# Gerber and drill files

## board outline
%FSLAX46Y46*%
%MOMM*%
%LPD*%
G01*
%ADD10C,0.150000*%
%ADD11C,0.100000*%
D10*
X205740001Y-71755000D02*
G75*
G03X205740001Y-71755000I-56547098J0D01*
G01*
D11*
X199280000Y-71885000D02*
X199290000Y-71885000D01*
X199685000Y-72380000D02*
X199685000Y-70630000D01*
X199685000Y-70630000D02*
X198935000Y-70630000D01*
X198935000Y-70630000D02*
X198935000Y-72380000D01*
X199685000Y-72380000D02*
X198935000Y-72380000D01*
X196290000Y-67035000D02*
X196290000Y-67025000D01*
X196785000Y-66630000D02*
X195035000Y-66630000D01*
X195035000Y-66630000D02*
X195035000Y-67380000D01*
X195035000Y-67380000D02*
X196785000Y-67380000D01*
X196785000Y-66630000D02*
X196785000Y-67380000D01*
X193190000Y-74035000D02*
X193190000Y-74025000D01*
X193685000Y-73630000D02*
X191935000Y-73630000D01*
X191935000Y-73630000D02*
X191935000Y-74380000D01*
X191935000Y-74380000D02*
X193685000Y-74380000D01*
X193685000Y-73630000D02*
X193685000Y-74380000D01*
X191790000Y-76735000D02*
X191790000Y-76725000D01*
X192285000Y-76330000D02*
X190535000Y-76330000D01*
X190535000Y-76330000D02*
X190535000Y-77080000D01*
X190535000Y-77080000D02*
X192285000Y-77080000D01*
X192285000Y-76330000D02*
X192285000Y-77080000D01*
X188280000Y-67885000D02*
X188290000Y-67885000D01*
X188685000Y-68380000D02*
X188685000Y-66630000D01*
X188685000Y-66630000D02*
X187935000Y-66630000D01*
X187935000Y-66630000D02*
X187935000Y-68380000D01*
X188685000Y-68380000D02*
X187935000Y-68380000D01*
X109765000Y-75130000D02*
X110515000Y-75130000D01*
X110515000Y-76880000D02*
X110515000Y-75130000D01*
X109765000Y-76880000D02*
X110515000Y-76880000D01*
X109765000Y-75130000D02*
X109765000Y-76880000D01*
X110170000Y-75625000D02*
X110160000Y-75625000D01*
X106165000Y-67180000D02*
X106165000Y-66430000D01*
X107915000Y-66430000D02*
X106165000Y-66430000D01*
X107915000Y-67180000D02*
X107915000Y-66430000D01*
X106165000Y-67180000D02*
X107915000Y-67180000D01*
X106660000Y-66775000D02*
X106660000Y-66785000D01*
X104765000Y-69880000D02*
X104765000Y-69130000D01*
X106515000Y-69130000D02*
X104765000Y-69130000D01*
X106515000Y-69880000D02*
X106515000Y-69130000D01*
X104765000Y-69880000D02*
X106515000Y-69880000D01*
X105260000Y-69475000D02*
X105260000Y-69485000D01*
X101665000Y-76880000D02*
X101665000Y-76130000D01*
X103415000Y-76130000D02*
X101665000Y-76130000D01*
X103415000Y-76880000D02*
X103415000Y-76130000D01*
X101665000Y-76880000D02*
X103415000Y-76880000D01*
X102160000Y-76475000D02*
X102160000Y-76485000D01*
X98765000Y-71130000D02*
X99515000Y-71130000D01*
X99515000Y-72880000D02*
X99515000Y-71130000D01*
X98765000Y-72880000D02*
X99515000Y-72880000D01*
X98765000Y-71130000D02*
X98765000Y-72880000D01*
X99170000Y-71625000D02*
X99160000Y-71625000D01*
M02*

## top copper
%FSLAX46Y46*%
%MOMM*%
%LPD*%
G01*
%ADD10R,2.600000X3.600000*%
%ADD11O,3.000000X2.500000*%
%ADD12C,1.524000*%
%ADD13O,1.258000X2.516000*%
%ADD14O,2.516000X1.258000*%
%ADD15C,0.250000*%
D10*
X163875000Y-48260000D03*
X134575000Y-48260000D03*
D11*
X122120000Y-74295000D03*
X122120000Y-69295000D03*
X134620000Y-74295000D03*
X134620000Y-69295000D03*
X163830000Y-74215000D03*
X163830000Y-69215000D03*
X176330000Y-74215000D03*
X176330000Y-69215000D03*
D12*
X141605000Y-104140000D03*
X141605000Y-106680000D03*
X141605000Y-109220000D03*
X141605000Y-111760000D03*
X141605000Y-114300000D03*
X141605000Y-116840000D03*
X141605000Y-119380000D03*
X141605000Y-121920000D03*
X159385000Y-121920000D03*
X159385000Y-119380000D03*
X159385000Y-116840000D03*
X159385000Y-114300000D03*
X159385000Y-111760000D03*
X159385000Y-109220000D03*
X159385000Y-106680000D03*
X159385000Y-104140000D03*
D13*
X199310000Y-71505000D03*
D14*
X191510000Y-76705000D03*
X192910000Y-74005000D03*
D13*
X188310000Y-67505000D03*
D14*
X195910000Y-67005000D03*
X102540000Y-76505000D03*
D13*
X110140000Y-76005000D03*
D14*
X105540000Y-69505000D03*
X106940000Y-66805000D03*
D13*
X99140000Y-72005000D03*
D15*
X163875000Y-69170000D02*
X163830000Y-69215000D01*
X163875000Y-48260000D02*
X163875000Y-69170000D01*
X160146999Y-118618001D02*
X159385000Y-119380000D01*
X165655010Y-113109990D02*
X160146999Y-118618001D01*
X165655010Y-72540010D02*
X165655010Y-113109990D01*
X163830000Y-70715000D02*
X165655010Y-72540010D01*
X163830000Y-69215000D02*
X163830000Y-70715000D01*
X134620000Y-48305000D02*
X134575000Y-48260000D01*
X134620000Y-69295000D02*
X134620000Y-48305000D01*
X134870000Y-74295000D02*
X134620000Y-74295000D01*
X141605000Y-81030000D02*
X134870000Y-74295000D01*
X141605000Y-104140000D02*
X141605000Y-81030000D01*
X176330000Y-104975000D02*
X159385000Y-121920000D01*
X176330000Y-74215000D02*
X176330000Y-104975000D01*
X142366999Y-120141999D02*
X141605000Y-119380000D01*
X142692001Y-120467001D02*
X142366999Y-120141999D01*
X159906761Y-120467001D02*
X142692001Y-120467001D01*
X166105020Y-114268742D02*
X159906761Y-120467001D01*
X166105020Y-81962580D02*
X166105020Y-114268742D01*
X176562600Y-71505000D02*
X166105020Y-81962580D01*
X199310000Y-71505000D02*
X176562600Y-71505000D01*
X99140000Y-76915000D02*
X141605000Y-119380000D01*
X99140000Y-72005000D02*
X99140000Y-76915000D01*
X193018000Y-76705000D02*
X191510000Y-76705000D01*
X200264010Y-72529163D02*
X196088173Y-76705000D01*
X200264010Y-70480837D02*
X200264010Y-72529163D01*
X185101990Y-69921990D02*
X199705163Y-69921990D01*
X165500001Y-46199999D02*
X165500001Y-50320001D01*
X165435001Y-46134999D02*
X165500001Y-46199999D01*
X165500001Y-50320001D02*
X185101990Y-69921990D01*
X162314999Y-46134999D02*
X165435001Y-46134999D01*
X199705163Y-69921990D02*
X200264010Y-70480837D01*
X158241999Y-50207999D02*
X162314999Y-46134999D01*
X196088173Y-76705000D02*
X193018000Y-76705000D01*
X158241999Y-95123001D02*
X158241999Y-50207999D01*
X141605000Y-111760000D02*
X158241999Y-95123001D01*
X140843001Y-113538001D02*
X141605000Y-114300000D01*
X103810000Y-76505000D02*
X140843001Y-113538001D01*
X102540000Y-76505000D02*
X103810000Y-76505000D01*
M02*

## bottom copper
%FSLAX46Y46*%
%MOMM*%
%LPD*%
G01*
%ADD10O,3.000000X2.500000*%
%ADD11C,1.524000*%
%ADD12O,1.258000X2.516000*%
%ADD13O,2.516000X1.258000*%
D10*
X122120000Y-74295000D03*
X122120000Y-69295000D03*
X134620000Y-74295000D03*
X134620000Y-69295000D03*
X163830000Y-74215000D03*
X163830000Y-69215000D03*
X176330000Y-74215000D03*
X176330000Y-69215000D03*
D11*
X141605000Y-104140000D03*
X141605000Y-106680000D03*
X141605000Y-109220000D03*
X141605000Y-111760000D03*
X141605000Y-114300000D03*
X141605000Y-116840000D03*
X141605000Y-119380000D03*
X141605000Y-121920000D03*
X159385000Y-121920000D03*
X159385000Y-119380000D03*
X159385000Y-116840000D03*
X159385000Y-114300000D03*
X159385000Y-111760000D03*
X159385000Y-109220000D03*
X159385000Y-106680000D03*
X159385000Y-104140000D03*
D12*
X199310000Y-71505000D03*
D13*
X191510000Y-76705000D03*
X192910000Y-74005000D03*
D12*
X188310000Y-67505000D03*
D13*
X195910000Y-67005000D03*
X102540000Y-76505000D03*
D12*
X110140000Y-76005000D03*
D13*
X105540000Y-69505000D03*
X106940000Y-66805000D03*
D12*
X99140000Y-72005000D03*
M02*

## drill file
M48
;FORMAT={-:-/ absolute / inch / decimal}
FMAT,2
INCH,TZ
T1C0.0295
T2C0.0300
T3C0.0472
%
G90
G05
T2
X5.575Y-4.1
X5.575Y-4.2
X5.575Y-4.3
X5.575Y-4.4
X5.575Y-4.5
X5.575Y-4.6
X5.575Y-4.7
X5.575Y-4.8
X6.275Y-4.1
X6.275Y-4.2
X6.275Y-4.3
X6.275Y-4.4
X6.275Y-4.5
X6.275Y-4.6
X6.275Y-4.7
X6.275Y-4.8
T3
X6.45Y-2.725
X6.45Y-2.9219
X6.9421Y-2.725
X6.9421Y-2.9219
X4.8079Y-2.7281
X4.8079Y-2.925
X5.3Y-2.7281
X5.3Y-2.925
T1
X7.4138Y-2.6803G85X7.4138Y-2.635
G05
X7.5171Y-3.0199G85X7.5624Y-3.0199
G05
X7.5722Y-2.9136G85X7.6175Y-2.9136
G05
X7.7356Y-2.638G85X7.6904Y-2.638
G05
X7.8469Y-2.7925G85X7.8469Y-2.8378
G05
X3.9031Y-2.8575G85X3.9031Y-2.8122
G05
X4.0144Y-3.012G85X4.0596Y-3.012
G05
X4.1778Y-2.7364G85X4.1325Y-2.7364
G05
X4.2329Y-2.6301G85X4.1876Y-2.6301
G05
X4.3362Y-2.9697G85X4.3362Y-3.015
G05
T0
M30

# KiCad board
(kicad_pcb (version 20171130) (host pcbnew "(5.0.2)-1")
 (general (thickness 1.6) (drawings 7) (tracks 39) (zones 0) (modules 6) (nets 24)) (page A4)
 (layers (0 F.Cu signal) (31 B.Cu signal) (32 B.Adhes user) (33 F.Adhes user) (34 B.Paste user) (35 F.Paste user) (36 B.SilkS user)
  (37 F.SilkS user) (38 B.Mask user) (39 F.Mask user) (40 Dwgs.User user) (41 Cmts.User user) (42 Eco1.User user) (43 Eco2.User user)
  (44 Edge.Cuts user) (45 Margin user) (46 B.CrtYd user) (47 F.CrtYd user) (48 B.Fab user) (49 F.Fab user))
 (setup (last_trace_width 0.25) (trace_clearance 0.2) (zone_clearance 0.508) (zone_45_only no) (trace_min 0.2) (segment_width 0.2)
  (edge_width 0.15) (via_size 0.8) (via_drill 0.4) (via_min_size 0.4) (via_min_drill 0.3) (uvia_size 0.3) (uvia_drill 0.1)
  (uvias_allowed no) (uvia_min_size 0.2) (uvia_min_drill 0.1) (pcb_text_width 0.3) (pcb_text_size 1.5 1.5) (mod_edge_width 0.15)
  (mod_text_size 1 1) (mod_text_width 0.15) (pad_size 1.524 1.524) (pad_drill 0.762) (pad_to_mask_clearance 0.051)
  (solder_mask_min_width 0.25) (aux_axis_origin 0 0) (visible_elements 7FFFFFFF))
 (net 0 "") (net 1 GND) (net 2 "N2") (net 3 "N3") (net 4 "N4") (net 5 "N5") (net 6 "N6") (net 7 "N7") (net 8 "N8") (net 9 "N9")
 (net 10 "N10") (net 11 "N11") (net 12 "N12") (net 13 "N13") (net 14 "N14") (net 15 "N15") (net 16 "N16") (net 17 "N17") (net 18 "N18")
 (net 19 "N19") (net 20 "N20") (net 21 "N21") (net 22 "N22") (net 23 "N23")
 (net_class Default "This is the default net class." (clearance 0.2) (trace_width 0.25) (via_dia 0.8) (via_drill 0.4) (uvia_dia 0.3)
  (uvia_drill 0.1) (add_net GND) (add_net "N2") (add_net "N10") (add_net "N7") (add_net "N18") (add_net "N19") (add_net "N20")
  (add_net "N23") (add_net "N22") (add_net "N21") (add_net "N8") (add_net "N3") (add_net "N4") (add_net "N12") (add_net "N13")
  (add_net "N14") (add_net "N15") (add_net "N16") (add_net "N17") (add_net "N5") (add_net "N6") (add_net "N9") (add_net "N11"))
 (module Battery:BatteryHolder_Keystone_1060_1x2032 (layer F.Cu) (at 149.225 48.26)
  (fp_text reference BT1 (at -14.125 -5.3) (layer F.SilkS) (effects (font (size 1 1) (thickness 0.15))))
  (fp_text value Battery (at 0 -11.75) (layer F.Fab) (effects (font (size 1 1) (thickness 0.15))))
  (pad 2 smd rect (at 14.65 0 180) (size 2.6 3.6) (layers F.Cu F.Paste F.Mask) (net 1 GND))
  (pad 1 smd rect (at -14.65 0 180) (size 2.6 3.6) (layers F.Cu F.Paste F.Mask) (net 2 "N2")))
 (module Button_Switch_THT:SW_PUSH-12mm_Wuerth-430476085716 (layer F.Cu) (at 134.62 74.295 180)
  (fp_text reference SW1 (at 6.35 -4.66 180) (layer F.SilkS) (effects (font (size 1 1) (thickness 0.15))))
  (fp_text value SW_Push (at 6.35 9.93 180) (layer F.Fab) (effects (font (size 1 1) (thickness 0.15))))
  (pad 1 thru_hole oval (at 12.5 0 180) (size 3 2.5) (drill 1.2) (layers *.Cu *.Mask) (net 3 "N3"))
  (pad 2 thru_hole oval (at 12.5 5 180) (size 3 2.5) (drill 1.2) (layers *.Cu *.Mask) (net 2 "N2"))
  (pad 1 thru_hole oval (at 0 0 180) (size 3 2.5) (drill 1.2) (layers *.Cu *.Mask) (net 3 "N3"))
  (pad 2 thru_hole oval (at 0 5 180) (size 3 2.5) (drill 1.2) (layers *.Cu *.Mask) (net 2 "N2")))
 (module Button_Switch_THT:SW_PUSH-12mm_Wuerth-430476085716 (layer F.Cu) (at 163.83 69.215)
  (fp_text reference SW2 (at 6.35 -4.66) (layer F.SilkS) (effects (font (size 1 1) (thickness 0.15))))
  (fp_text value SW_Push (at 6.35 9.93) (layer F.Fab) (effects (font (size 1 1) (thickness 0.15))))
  (pad 2 thru_hole oval (at 0 5) (size 3 2.5) (drill 1.2) (layers *.Cu *.Mask) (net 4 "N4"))
  (pad 1 thru_hole oval (at 0 0) (size 3 2.5) (drill 1.2) (layers *.Cu *.Mask) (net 1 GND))
  (pad 2 thru_hole oval (at 12.5 5) (size 3 2.5) (drill 1.2) (layers *.Cu *.Mask) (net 4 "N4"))
  (pad 1 thru_hole oval (at 12.5 0) (size 3 2.5) (drill 1.2) (layers *.Cu *.Mask) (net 1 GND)))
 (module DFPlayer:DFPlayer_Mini (layer F.Cu) (at 150.495 101.6)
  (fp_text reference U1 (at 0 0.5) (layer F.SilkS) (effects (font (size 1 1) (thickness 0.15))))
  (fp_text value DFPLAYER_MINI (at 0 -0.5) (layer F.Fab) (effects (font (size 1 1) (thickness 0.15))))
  (pad 1 thru_hole circle (at -8.89 2.54) (size 1.524 1.524) (drill 0.762) (layers *.Cu *.Mask) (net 3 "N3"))
  (pad 2 thru_hole circle (at -8.89 5.08) (size 1.524 1.524) (drill 0.762) (layers *.Cu *.Mask) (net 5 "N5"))
  (pad 3 thru_hole circle (at -8.89 7.62) (size 1.524 1.524) (drill 0.762) (layers *.Cu *.Mask) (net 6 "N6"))
  (pad 4 thru_hole circle (at -8.89 10.16) (size 1.524 1.524) (drill 0.762) (layers *.Cu *.Mask) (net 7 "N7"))
  (pad 5 thru_hole circle (at -8.89 12.7) (size 1.524 1.524) (drill 0.762) (layers *.Cu *.Mask) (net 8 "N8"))
  (pad 6 thru_hole circle (at -8.89 15.24) (size 1.524 1.524) (drill 0.762) (layers *.Cu *.Mask) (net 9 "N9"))
  (pad 7 thru_hole circle (at -8.89 17.78) (size 1.524 1.524) (drill 0.762) (layers *.Cu *.Mask) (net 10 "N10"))
  (pad 8 thru_hole circle (at -8.89 20.32) (size 1.524 1.524) (drill 0.762) (layers *.Cu *.Mask) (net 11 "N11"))
  (pad 9 thru_hole circle (at 8.89 20.32) (size 1.524 1.524) (drill 0.762) (layers *.Cu *.Mask) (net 4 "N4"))
  (pad 10 thru_hole circle (at 8.89 17.78) (size 1.524 1.524) (drill 0.762) (layers *.Cu *.Mask) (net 1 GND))
  (pad 11 thru_hole circle (at 8.89 15.24) (size 1.524 1.524) (drill 0.762) (layers *.Cu *.Mask) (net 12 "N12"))
  (pad 12 thru_hole circle (at 8.89 12.7) (size 1.524 1.524) (drill 0.762) (layers *.Cu *.Mask) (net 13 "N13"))
  (pad 13 thru_hole circle (at 8.89 10.16) (size 1.524 1.524) (drill 0.762) (layers *.Cu *.Mask) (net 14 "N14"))
  (pad 14 thru_hole circle (at 8.89 7.62) (size 1.524 1.524) (drill 0.762) (layers *.Cu *.Mask) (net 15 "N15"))
  (pad 15 thru_hole circle (at 8.89 5.08) (size 1.524 1.524) (drill 0.762) (layers *.Cu *.Mask) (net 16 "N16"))
  (pad 16 thru_hole circle (at 8.89 2.54) (size 1.524 1.524) (drill 0.762) (layers *.Cu *.Mask) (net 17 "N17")))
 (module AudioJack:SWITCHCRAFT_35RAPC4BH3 (layer F.Cu) (at 194.31 71.755 180)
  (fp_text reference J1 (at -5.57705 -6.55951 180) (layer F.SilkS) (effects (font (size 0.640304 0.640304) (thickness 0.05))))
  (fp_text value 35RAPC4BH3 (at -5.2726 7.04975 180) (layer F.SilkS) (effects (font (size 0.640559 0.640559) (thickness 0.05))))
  (fp_line (start -4.97 -0.13) (end -4.98 -0.13) (layer Edge.Cuts) (width 0.1))
  (fp_line (start -5.375 -0.625) (end -5.375 1.125) (layer Edge.Cuts) (width 0.1))
  (fp_line (start -5.375 1.125) (end -4.625 1.125) (layer Edge.Cuts) (width 0.1))
  (fp_line (start -4.625 1.125) (end -4.625 -0.625) (layer Edge.Cuts) (width 0.1))
  (fp_line (start -5.375 -0.625) (end -4.625 -0.625) (layer Edge.Cuts) (width 0.1))
  (fp_line (start -1.98 4.72) (end -1.98 4.73) (layer Edge.Cuts) (width 0.1))
  (fp_line (start -2.475 5.125) (end -0.725 5.125) (layer Edge.Cuts) (width 0.1))
  (fp_line (start -0.725 5.125) (end -0.725 4.375) (layer Edge.Cuts) (width 0.1))
  (fp_line (start -0.725 4.375) (end -2.475 4.375) (layer Edge.Cuts) (width 0.1))
  (fp_line (start -2.475 5.125) (end -2.475 4.375) (layer Edge.Cuts) (width 0.1))
  (fp_line (start 1.12 -2.28) (end 1.12 -2.27) (layer Edge.Cuts) (width 0.1))
  (fp_line (start 0.625 -1.875) (end 2.375 -1.875) (layer Edge.Cuts) (width 0.1))
  (fp_line (start 2.375 -1.875) (end 2.375 -2.625) (layer Edge.Cuts) (width 0.1))
  (fp_line (start 2.375 -2.625) (end 0.625 -2.625) (layer Edge.Cuts) (width 0.1))
  (fp_line (start 0.625 -1.875) (end 0.625 -2.625) (layer Edge.Cuts) (width 0.1))
  (fp_line (start 2.52 -4.98) (end 2.52 -4.97) (layer Edge.Cuts) (width 0.1))
  (fp_line (start 2.025 -4.575) (end 3.775 -4.575) (layer Edge.Cuts) (width 0.1))
  (fp_line (start 3.775 -4.575) (end 3.775 -5.325) (layer Edge.Cuts) (width 0.1))
  (fp_line (start 3.775 -5.325) (end 2.025 -5.325) (layer Edge.Cuts) (width 0.1))
  (fp_line (start 2.025 -4.575) (end 2.025 -5.325) (layer Edge.Cuts) (width 0.1))
  (fp_line (start 6.03 3.87) (end 6.02 3.87) (layer Edge.Cuts) (width 0.1))
  (fp_line (start 5.625 3.375) (end 5.625 5.125) (layer Edge.Cuts) (width 0.1))
  (fp_line (start 5.625 5.125) (end 6.375 5.125) (layer Edge.Cuts) (width 0.1))
  (fp_line (start 6.375 5.125) (end 6.375 3.375) (layer Edge.Cuts) (width 0.1))
  (fp_line (start 5.625 3.375) (end 6.375 3.375) (layer Edge.Cuts) (width 0.1))
  (pad 1 thru_hole oval (at -5 0.25 270) (size 2.516 1.258) (drill oval 1.9 0.75) (layers *.Cu *.Mask) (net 10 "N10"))
  (pad 2 thru_hole oval (at 2.8 -4.95) (size 2.516 1.258) (drill oval 1.9 0.75) (layers *.Cu *.Mask) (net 7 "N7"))
  (pad 3 thru_hole oval (at 1.4 -2.25) (size 2.516 1.258) (drill oval 1.9 0.75) (layers *.Cu *.Mask) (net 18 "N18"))
  (pad 4 thru_hole oval (at 6 4.25 90) (size 2.516 1.258) (drill oval 1.9 0.75) (layers *.Cu *.Mask) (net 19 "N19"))
  (pad 5 thru_hole oval (at -1.6 4.75 180) (size 2.516 1.258) (drill oval 1.9 0.75) (layers *.Cu *.Mask) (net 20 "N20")))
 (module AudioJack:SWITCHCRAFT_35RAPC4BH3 (layer F.Cu) (at 104.14 71.755)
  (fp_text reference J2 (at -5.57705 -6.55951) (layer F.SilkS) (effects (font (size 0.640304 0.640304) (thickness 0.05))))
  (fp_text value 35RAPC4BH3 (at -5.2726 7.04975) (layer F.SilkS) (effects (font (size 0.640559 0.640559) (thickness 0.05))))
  (fp_line (start 5.625 3.375) (end 6.375 3.375) (layer Edge.Cuts) (width 0.1))
  (fp_line (start 6.375 5.125) (end 6.375 3.375) (layer Edge.Cuts) (width 0.1))
  (fp_line (start 5.625 5.125) (end 6.375 5.125) (layer Edge.Cuts) (width 0.1))
  (fp_line (start 5.625 3.375) (end 5.625 5.125) (layer Edge.Cuts) (width 0.1))
  (fp_line (start 6.03 3.87) (end 6.02 3.87) (layer Edge.Cuts) (width 0.1))
  (fp_line (start 2.025 -4.575) (end 2.025 -5.325) (layer Edge.Cuts) (width 0.1))
  (fp_line (start 3.775 -5.325) (end 2.025 -5.325) (layer Edge.Cuts) (width 0.1))
  (fp_line (start 3.775 -4.575) (end 3.775 -5.325) (layer Edge.Cuts) (width 0.1))
  (fp_line (start 2.025 -4.575) (end 3.775 -4.575) (layer Edge.Cuts) (width 0.1))
  (fp_line (start 2.52 -4.98) (end 2.52 -4.97) (layer Edge.Cuts) (width 0.1))
  (fp_line (start 0.625 -1.875) (end 0.625 -2.625) (layer Edge.Cuts) (width 0.1))
  (fp_line (start 2.375 -2.625) (end 0.625 -2.625) (layer Edge.Cuts) (width 0.1))
  (fp_line (start 2.375 -1.875) (end 2.375 -2.625) (layer Edge.Cuts) (width 0.1))
  (fp_line (start 0.625 -1.875) (end 2.375 -1.875) (layer Edge.Cuts) (width 0.1))
  (fp_line (start 1.12 -2.28) (end 1.12 -2.27) (layer Edge.Cuts) (width 0.1))
  (fp_line (start -2.475 5.125) (end -2.475 4.375) (layer Edge.Cuts) (width 0.1))
  (fp_line (start -0.725 4.375) (end -2.475 4.375) (layer Edge.Cuts) (width 0.1))
  (fp_line (start -0.725 5.125) (end -0.725 4.375) (layer Edge.Cuts) (width 0.1))
  (fp_line (start -2.475 5.125) (end -0.725 5.125) (layer Edge.Cuts) (width 0.1))
  (fp_line (start -1.98 4.72) (end -1.98 4.73) (layer Edge.Cuts) (width 0.1))
  (fp_line (start -5.375 -0.625) (end -4.625 -0.625) (layer Edge.Cuts) (width 0.1))
  (fp_line (start -4.625 1.125) (end -4.625 -0.625) (layer Edge.Cuts) (width 0.1))
  (fp_line (start -5.375 1.125) (end -4.625 1.125) (layer Edge.Cuts) (width 0.1))
  (fp_line (start -5.375 -0.625) (end -5.375 1.125) (layer Edge.Cuts) (width 0.1))
  (fp_line (start -4.97 -0.13) (end -4.98 -0.13) (layer Edge.Cuts) (width 0.1))
  (pad 5 thru_hole oval (at -1.6 4.75) (size 2.516 1.258) (drill oval 1.9 0.75) (layers *.Cu *.Mask) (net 8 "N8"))
  (pad 4 thru_hole oval (at 6 4.25 270) (size 2.516 1.258) (drill oval 1.9 0.75) (layers *.Cu *.Mask) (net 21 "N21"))
  (pad 3 thru_hole oval (at 1.4 -2.25 180) (size 2.516 1.258) (drill oval 1.9 0.75) (layers *.Cu *.Mask) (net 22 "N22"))
  (pad 2 thru_hole oval (at 2.8 -4.95 180) (size 2.516 1.258) (drill oval 1.9 0.75) (layers *.Cu *.Mask) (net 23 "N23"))
  (pad 1 thru_hole oval (at -5 0.25 90) (size 2.516 1.258) (drill oval 1.9 0.75) (layers *.Cu *.Mask) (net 10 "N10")))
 (gr_circle (center 149.192903 71.755) (end 147.287903 15.24) (layer Edge.Cuts) (width 0.15))
 (segment (start 163.875 69.17) (end 163.83 69.215) (width 0.25) (layer F.Cu) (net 1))
 (segment (start 163.875 48.26) (end 163.875 69.17) (width 0.25) (layer F.Cu) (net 1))
 (segment (start 160.146999 118.618001) (end 159.385 119.38) (width 0.25) (layer F.Cu) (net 1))
 (segment (start 165.65501 113.10999) (end 160.146999 118.618001) (width 0.25) (layer F.Cu) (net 1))
 (segment (start 165.65501 72.54001) (end 165.65501 113.10999) (width 0.25) (layer F.Cu) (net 1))
 (segment (start 163.83 70.715) (end 165.65501 72.54001) (width 0.25) (layer F.Cu) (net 1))
 (segment (start 163.83 69.215) (end 163.83 70.715) (width 0.25) (layer F.Cu) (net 1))
 (segment (start 134.62 48.305) (end 134.575 48.26) (width 0.25) (layer F.Cu) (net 2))
 (segment (start 134.62 69.295) (end 134.62 48.305) (width 0.25) (layer F.Cu) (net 2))
 (segment (start 134.87 74.295) (end 134.62 74.295) (width 0.25) (layer F.Cu) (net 3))
 (segment (start 141.605 81.03) (end 134.87 74.295) (width 0.25) (layer F.Cu) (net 3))
 (segment (start 141.605 104.14) (end 141.605 81.03) (width 0.25) (layer F.Cu) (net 3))
 (segment (start 176.33 104.975) (end 159.385 121.92) (width 0.25) (layer F.Cu) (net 4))
 (segment (start 176.33 74.215) (end 176.33 104.975) (width 0.25) (layer F.Cu) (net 4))
 (segment (start 142.366999 120.141999) (end 141.605 119.38) (width 0.25) (layer F.Cu) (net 10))
 (segment (start 142.692001 120.467001) (end 142.366999 120.141999) (width 0.25) (layer F.Cu) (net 10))
 (segment (start 159.906761 120.467001) (end 142.692001 120.467001) (width 0.25) (layer F.Cu) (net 10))
 (segment (start 166.10502 114.268742) (end 159.906761 120.467001) (width 0.25) (layer F.Cu) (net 10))
 (segment (start 166.10502 81.96258) (end 166.10502 114.268742) (width 0.25) (layer F.Cu) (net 10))
 (segment (start 176.5626 71.505) (end 166.10502 81.96258) (width 0.25) (layer F.Cu) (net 10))
 (segment (start 199.31 71.505) (end 176.5626 71.505) (width 0.25) (layer F.Cu) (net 10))
 (segment (start 99.14 76.915) (end 141.605 119.38) (width 0.25) (layer F.Cu) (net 10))
 (segment (start 99.14 72.005) (end 99.14 76.915) (width 0.25) (layer F.Cu) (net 10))
 (segment (start 193.018 76.705) (end 191.51 76.705) (width 0.25) (layer F.Cu) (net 7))
 (segment (start 200.26401 72.529163) (end 196.088173 76.705) (width 0.25) (layer F.Cu) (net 7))
 (segment (start 200.26401 70.480837) (end 200.26401 72.529163) (width 0.25) (layer F.Cu) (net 7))
 (segment (start 185.10199 69.92199) (end 199.705163 69.92199) (width 0.25) (layer F.Cu) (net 7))
 (segment (start 165.500001 46.199999) (end 165.500001 50.320001) (width 0.25) (layer F.Cu) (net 7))
 (segment (start 165.435001 46.134999) (end 165.500001 46.199999) (width 0.25) (layer F.Cu) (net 7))
 (segment (start 165.500001 50.320001) (end 185.10199 69.92199) (width 0.25) (layer F.Cu) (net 7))
 (segment (start 162.314999 46.134999) (end 165.435001 46.134999) (width 0.25) (layer F.Cu) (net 7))
 (segment (start 199.705163 69.92199) (end 200.26401 70.480837) (width 0.25) (layer F.Cu) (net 7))
 (segment (start 158.241999 50.207999) (end 162.314999 46.134999) (width 0.25) (layer F.Cu) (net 7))
 (segment (start 196.088173 76.705) (end 193.018 76.705) (width 0.25) (layer F.Cu) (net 7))
 (segment (start 158.241999 95.123001) (end 158.241999 50.207999) (width 0.25) (layer F.Cu) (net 7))
 (segment (start 141.605 111.76) (end 158.241999 95.123001) (width 0.25) (layer F.Cu) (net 7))
 (segment (start 140.843001 113.538001) (end 141.605 114.3) (width 0.25) (layer F.Cu) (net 8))
 (segment (start 103.81 76.505) (end 140.843001 113.538001) (width 0.25) (layer F.Cu) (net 8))
 (segment (start 102.54 76.505) (end 103.81 76.505) (width 0.25) (layer F.Cu) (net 8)))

